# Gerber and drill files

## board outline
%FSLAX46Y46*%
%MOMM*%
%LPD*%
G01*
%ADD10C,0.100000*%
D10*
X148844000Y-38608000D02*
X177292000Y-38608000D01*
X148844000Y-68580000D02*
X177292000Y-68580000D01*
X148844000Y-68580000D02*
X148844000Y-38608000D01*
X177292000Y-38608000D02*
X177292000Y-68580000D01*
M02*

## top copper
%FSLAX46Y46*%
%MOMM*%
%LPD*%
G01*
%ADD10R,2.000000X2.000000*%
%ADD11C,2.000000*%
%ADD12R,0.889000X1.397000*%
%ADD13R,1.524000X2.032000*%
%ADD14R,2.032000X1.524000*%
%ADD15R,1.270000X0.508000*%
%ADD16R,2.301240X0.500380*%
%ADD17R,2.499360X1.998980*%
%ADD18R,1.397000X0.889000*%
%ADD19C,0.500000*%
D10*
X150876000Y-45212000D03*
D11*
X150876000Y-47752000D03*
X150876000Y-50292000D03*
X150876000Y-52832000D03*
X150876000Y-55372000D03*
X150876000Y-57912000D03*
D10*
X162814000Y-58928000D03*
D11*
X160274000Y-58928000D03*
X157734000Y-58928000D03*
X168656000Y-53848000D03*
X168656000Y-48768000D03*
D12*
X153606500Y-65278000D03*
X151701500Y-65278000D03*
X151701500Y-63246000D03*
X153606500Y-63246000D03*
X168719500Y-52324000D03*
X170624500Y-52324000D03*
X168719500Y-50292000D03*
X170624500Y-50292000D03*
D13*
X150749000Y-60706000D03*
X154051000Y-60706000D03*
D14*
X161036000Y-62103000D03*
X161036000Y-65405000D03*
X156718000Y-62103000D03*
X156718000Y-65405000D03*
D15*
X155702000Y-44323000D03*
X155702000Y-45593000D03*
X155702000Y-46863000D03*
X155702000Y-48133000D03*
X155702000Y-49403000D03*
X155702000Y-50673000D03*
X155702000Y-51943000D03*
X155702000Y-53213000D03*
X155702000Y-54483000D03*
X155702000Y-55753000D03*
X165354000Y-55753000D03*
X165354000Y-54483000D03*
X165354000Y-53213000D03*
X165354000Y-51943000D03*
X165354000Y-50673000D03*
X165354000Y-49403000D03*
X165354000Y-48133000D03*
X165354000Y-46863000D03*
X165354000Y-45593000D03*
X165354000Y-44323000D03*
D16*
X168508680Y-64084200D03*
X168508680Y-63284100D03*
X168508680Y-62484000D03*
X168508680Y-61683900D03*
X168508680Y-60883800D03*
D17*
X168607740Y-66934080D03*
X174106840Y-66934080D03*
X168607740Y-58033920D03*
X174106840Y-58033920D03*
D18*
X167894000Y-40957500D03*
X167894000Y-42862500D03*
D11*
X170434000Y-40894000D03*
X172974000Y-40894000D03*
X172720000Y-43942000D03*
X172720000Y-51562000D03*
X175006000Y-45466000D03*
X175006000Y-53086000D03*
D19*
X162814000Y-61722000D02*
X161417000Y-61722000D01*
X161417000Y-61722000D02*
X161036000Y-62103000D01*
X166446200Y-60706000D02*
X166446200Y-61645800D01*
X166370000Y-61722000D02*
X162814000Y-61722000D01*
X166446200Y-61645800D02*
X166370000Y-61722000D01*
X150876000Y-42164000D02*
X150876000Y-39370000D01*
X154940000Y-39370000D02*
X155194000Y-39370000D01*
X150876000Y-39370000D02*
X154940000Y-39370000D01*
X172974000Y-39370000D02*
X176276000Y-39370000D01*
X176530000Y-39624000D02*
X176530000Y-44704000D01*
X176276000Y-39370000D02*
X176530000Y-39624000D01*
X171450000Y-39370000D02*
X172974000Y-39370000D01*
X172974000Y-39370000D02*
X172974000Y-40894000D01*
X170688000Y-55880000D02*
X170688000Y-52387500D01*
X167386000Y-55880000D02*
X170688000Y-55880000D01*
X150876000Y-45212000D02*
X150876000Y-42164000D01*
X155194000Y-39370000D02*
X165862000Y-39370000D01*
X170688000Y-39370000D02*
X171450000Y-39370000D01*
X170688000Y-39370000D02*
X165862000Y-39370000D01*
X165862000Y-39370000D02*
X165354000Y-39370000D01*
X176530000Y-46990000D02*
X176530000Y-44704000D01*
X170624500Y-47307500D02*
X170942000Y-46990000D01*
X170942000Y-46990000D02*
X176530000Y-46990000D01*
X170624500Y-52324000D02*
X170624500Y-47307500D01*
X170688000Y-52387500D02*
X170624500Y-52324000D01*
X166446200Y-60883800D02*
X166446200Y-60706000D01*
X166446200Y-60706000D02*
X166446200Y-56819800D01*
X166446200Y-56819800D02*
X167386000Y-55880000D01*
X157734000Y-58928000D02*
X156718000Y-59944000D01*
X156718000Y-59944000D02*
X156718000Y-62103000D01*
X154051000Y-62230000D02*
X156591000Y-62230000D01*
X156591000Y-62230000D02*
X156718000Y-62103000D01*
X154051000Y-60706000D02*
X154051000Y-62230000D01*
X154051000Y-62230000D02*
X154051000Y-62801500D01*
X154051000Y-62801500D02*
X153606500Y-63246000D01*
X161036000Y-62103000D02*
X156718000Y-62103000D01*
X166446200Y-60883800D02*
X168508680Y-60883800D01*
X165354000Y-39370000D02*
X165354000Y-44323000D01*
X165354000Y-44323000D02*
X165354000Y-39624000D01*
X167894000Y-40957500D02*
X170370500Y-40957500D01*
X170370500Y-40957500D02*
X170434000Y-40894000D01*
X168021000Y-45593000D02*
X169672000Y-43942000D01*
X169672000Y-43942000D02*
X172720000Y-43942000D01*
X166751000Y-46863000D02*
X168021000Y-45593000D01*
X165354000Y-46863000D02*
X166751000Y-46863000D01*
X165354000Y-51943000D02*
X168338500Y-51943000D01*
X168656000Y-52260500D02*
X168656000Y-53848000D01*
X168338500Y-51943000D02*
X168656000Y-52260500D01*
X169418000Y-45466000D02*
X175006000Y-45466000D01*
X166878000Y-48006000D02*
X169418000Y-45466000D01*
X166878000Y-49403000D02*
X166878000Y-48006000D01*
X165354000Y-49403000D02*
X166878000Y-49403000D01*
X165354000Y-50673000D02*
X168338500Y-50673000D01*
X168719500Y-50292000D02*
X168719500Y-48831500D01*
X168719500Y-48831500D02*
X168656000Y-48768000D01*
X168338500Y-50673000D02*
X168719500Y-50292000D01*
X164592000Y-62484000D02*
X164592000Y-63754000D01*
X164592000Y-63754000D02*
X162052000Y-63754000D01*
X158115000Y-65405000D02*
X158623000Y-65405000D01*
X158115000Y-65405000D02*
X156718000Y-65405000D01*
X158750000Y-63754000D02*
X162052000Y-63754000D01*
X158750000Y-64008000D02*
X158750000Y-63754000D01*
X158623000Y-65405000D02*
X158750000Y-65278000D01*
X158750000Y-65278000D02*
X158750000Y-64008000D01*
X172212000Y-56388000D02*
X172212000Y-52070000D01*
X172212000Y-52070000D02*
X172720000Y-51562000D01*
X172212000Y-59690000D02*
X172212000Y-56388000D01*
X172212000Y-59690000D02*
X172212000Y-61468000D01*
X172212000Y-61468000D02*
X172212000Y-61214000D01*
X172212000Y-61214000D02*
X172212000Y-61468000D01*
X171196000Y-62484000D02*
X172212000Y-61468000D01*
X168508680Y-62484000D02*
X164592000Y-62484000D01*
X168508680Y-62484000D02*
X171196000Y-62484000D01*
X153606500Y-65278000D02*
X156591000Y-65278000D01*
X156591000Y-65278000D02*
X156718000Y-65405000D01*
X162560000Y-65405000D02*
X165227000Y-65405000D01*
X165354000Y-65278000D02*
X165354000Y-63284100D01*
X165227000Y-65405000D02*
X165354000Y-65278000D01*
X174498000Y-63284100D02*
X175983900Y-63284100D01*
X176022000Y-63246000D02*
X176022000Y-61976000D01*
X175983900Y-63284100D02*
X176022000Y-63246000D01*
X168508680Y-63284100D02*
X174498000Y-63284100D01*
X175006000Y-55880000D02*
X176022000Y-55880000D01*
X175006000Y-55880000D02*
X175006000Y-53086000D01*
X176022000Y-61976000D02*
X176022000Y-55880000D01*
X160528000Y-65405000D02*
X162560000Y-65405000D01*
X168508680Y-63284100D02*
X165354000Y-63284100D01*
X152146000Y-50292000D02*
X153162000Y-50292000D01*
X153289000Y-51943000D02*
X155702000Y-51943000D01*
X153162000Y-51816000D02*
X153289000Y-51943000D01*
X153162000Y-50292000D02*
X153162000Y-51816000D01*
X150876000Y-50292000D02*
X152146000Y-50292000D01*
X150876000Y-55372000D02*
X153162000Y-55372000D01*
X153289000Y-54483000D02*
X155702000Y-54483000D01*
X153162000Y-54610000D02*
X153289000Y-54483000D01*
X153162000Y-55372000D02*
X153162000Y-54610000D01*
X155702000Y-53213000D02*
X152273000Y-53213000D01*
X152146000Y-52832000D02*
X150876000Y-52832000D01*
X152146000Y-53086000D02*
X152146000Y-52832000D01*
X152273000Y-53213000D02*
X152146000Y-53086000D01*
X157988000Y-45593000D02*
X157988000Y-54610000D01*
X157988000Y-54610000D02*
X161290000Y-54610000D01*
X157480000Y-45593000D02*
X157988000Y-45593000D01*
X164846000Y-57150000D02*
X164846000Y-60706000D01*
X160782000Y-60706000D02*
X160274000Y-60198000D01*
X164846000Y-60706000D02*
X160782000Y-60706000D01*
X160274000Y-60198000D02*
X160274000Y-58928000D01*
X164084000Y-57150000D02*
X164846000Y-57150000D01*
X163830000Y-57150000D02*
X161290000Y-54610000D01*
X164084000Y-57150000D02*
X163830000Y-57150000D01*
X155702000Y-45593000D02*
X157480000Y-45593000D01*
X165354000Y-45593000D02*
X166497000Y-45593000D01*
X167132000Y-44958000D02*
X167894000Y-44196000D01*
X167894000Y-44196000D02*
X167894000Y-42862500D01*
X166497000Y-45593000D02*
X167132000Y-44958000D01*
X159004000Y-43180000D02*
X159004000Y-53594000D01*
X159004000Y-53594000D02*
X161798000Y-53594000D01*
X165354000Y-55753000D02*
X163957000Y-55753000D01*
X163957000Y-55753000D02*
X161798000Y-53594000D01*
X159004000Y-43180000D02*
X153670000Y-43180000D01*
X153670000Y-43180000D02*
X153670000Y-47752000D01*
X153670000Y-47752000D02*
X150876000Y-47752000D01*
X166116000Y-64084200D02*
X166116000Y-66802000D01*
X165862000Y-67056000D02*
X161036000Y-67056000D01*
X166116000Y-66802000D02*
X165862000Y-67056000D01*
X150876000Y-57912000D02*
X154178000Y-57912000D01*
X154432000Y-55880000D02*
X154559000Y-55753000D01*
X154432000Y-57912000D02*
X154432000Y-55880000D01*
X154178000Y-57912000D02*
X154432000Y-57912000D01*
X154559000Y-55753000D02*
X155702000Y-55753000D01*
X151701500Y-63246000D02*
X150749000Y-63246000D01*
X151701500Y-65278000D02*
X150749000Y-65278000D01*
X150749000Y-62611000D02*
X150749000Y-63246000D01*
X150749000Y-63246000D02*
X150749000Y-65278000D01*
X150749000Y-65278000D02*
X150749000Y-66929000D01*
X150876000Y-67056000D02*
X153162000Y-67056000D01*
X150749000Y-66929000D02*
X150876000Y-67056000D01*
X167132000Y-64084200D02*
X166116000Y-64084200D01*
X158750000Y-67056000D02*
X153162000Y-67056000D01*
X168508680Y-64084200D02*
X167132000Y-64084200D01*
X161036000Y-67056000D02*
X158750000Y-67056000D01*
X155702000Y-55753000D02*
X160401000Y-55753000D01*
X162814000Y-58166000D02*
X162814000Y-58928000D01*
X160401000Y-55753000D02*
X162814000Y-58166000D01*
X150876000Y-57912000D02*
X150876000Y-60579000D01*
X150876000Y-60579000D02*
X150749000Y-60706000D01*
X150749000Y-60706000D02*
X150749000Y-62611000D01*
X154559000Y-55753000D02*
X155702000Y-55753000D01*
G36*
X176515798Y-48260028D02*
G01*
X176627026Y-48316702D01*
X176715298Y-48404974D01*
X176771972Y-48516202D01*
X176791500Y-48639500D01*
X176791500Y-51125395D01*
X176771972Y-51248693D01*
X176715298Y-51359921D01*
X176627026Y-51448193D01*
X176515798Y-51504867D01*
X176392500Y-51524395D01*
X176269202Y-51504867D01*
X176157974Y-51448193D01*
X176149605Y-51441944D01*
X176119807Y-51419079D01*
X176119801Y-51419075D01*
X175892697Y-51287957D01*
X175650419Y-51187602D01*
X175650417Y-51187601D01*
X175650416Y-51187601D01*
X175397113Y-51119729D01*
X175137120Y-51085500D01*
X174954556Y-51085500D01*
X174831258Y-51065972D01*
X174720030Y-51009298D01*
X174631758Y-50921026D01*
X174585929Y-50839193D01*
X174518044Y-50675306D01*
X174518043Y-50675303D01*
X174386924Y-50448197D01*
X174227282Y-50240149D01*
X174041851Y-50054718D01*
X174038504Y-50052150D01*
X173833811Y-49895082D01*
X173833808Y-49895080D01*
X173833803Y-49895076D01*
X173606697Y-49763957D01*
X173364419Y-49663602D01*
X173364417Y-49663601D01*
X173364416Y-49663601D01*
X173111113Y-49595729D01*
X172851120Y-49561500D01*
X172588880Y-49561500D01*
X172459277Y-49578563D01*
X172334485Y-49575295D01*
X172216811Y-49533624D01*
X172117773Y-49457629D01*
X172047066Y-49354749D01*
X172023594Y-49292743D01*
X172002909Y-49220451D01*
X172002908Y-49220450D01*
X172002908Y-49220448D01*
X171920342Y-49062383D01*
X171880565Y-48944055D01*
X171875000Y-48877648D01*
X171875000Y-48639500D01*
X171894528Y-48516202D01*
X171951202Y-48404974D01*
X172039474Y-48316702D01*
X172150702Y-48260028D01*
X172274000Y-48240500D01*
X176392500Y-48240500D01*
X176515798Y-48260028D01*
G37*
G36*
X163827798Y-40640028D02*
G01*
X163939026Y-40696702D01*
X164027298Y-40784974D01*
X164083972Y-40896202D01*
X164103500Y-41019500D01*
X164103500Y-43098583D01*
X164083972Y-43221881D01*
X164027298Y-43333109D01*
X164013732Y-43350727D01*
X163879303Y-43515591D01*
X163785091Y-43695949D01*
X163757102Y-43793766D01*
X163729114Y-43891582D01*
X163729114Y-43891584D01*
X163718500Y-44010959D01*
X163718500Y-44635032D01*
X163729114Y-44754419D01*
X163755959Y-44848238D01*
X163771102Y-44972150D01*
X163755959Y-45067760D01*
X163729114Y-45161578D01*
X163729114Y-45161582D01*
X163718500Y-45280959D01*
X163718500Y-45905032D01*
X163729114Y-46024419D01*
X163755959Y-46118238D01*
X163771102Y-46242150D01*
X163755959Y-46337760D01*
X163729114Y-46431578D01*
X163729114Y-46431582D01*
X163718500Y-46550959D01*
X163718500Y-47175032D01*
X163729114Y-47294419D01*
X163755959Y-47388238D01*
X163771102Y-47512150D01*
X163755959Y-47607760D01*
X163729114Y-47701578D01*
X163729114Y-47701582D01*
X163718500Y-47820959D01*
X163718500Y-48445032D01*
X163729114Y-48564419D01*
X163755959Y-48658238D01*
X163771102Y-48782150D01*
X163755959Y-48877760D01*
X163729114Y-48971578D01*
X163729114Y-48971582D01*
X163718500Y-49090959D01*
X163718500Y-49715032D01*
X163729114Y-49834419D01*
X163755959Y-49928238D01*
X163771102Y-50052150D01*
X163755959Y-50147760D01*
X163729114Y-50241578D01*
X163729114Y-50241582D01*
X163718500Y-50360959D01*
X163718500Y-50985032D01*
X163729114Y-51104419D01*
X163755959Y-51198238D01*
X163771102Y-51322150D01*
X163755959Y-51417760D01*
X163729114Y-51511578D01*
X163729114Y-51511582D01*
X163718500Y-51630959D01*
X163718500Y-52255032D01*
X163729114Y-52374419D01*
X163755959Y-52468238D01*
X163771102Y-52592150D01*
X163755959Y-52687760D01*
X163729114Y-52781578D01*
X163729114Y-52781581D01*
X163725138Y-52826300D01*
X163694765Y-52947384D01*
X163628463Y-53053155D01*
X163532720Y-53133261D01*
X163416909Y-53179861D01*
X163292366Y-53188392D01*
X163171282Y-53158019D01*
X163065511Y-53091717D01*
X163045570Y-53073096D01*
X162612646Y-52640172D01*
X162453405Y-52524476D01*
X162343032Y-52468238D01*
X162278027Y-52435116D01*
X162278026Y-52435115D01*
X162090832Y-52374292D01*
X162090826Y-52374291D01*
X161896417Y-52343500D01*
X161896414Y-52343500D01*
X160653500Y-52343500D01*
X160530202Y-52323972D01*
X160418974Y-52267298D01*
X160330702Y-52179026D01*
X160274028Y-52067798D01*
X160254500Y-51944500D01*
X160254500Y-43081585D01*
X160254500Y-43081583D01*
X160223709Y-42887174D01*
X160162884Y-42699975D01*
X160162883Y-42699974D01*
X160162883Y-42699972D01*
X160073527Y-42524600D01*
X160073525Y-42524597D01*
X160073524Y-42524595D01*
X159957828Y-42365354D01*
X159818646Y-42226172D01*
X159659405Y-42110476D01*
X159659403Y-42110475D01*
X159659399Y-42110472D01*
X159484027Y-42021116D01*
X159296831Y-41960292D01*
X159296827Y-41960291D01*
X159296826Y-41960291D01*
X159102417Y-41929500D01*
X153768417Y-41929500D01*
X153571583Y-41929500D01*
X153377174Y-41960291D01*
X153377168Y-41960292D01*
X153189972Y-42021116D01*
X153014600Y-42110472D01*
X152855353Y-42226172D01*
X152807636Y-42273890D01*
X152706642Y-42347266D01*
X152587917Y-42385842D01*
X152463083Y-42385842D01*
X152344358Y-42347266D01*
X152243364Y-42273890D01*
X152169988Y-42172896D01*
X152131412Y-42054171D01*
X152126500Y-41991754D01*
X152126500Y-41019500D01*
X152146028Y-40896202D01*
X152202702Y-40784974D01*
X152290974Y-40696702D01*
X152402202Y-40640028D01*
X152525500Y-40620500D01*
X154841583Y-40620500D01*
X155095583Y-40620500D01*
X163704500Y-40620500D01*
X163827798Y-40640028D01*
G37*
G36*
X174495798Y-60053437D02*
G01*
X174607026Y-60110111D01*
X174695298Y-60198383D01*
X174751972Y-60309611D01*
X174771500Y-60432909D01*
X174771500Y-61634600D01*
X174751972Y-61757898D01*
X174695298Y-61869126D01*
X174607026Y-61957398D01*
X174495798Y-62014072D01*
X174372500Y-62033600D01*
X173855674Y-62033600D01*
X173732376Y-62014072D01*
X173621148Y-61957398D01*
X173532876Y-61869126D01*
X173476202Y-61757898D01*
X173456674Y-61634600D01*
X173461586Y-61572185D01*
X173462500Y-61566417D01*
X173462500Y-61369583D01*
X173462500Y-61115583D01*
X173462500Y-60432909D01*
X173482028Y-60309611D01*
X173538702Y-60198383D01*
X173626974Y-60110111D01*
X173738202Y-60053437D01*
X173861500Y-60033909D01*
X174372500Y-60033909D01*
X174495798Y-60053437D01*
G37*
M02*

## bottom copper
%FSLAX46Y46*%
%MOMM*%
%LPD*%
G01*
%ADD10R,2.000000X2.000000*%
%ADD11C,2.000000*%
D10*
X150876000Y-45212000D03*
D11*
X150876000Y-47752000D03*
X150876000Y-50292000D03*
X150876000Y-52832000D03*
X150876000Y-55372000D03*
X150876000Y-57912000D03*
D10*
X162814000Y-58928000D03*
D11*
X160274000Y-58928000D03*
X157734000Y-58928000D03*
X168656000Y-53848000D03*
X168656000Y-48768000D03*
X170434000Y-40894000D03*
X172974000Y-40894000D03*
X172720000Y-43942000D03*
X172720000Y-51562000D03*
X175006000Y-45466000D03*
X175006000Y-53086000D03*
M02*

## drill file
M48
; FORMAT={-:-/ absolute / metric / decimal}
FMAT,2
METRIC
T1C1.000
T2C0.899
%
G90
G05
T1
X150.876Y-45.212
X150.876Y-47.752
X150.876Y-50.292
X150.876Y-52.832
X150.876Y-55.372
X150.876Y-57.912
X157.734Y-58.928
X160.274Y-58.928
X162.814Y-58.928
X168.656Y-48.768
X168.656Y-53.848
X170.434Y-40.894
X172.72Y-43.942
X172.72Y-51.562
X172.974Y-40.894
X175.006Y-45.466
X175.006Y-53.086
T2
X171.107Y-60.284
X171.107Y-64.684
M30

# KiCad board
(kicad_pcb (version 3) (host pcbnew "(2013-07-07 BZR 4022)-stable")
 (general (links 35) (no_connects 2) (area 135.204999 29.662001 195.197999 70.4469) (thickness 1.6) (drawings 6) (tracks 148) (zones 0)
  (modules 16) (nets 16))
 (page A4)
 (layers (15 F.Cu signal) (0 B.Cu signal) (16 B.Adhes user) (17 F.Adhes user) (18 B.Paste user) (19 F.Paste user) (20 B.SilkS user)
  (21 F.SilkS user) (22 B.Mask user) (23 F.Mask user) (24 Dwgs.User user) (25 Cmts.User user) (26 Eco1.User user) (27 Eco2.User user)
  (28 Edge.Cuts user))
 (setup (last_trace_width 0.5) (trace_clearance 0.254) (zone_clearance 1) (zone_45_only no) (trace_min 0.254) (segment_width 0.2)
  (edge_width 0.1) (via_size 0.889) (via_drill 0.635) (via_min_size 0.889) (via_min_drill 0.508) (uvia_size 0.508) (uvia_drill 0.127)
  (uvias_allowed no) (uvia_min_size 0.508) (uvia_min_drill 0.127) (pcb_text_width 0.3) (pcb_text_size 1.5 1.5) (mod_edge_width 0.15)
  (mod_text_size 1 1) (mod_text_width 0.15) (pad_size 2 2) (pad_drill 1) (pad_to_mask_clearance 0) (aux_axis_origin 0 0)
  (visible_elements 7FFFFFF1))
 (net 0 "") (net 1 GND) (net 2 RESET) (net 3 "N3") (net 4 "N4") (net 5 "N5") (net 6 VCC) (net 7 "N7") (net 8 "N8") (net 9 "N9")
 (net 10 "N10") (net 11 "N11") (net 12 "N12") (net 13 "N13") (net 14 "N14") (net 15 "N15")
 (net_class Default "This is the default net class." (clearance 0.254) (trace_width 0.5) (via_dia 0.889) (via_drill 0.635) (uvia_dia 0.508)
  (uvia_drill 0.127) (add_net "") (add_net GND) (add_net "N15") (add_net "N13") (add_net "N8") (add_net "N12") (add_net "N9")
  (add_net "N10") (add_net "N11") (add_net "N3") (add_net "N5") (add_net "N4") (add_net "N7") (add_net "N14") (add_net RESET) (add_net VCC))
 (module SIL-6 (layer B.Cu) (at 150.876 51.562 270)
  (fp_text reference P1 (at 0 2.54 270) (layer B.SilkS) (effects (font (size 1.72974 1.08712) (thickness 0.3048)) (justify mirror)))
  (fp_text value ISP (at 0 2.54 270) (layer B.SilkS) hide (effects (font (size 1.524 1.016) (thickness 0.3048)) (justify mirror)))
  (pad 1 thru_hole rect (at -6.35 0 270) (size 2 2) (drill 1) (layers *.Cu *.Mask B.SilkS) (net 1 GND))
  (pad 2 thru_hole circle (at -3.81 0 270) (size 2 2) (drill 1) (layers *.Cu *.Mask B.SilkS) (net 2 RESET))
  (pad 3 thru_hole circle (at -1.27 0 270) (size 2 2) (drill 1) (layers *.Cu *.Mask B.SilkS) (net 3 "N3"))
  (pad 4 thru_hole circle (at 1.27 0 270) (size 2 2) (drill 1) (layers *.Cu *.Mask B.SilkS) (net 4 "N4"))
  (pad 5 thru_hole circle (at 3.81 0 270) (size 2 2) (drill 1) (layers *.Cu *.Mask B.SilkS) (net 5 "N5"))
  (pad 6 thru_hole circle (at 6.35 0 270) (size 2 2) (drill 1) (layers *.Cu *.Mask B.SilkS) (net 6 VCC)))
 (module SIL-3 (layer B.Cu) (at 160.274 58.928 180)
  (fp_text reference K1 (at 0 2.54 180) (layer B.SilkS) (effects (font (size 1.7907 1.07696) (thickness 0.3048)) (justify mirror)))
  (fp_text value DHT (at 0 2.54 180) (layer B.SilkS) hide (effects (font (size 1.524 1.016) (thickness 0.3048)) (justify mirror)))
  (pad 1 thru_hole rect (at -2.54 0 180) (size 2 2) (drill 1) (layers *.Cu *.Mask B.SilkS) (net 6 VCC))
  (pad 2 thru_hole circle (at 0 0 180) (size 2 2) (drill 1) (layers *.Cu *.Mask B.SilkS) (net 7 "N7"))
  (pad 3 thru_hole circle (at 2.54 0 180) (size 2 2) (drill 1) (layers *.Cu *.Mask B.SilkS) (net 1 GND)))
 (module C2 (layer B.Cu) (at 168.656 51.308 90)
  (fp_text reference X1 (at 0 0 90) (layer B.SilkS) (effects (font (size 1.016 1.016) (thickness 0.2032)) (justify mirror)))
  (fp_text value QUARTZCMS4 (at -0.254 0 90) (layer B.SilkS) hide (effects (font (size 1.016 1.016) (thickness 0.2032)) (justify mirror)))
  (pad 1 thru_hole circle (at -2.54 0 90) (size 2 2) (drill 1) (layers *.Cu *.Mask B.SilkS) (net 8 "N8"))
  (pad 3 thru_hole circle (at 2.54 0 90) (size 2 2) (drill 1) (layers *.Cu *.Mask B.SilkS) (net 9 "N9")))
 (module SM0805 (layer F.Cu) (at 152.654 65.278 180)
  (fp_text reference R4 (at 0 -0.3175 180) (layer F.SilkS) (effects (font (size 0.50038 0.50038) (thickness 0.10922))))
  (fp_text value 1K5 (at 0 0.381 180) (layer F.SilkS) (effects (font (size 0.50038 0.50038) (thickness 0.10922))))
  (pad 1 smd rect (at -0.9525 0 180) (size 0.889 1.397) (layers F.Cu F.Paste F.Mask) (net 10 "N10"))
  (pad 2 smd rect (at 0.9525 0 180) (size 0.889 1.397) (layers F.Cu F.Paste F.Mask) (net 6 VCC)))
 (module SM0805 (layer F.Cu) (at 152.654 63.246)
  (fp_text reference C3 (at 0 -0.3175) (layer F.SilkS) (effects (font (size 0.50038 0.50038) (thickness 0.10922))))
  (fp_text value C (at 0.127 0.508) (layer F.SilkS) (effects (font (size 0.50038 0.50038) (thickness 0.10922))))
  (pad 1 smd rect (at -0.9525 0) (size 0.889 1.397) (layers F.Cu F.Paste F.Mask) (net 6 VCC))
  (pad 2 smd rect (at 0.9525 0) (size 0.889 1.397) (layers F.Cu F.Paste F.Mask) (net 1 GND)))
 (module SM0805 (layer F.Cu) (at 169.672 52.324)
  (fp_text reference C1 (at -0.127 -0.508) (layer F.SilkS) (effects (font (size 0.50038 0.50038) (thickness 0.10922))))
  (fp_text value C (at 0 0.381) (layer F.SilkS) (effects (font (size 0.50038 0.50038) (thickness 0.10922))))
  (pad 1 smd rect (at -0.9525 0) (size 0.889 1.397) (layers F.Cu F.Paste F.Mask) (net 8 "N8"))
  (pad 2 smd rect (at 0.9525 0) (size 0.889 1.397) (layers F.Cu F.Paste F.Mask) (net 1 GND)))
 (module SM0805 (layer F.Cu) (at 169.672 50.292)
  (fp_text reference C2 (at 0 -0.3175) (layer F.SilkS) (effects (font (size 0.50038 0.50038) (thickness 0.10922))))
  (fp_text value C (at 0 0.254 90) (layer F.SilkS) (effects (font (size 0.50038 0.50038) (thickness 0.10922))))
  (pad 1 smd rect (at -0.9525 0) (size 0.889 1.397) (layers F.Cu F.Paste F.Mask) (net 9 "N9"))
  (pad 2 smd rect (at 0.9525 0) (size 0.889 1.397) (layers F.Cu F.Paste F.Mask) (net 1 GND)))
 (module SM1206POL (layer F.Cu) (at 152.4 60.706)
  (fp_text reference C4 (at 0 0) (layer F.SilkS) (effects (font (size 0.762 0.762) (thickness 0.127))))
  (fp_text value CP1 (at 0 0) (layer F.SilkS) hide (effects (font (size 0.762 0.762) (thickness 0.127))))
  (pad 1 smd rect (at -1.651 0) (size 1.524 2.032) (layers F.Cu F.Paste F.Mask) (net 6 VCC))
  (pad 2 smd rect (at 1.651 0) (size 1.524 2.032) (layers F.Cu F.Paste F.Mask) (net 1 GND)))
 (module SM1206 (layer F.Cu) (at 161.036 63.754 270)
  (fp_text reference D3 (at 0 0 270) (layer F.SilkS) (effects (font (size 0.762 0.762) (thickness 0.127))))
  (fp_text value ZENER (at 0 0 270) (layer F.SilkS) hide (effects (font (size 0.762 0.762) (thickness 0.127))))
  (pad 1 smd rect (at -1.651 0 270) (size 1.524 2.032) (layers F.Cu F.Paste F.Mask) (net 1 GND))
  (pad 2 smd rect (at 1.651 0 270) (size 1.524 2.032) (layers F.Cu F.Paste F.Mask) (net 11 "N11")))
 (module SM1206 (layer F.Cu) (at 156.718 63.754 270)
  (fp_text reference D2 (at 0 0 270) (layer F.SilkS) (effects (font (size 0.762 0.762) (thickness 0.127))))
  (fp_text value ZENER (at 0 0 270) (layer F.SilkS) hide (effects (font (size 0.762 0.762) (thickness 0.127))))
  (pad 1 smd rect (at -1.651 0 270) (size 1.524 2.032) (layers F.Cu F.Paste F.Mask) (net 1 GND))
  (pad 2 smd rect (at 1.651 0 270) (size 1.524 2.032) (layers F.Cu F.Paste F.Mask) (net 10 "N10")))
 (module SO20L (layer F.Cu) (at 160.528 50.038 90)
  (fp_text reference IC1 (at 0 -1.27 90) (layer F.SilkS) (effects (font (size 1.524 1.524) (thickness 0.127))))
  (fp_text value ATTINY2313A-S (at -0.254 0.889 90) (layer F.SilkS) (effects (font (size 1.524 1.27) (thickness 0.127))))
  (pad 11 smd rect (at 5.715 -4.826 90) (size 0.508 1.27) (layers F.Cu F.Paste F.Mask))
  (pad 12 smd rect (at 4.445 -4.826 90) (size 0.508 1.27) (layers F.Cu F.Paste F.Mask) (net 7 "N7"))
  (pad 13 smd rect (at 3.175 -4.826 90) (size 0.508 1.27) (layers F.Cu F.Paste F.Mask))
  (pad 14 smd rect (at 1.905 -4.826 90) (size 0.508 1.27) (layers F.Cu F.Paste F.Mask))
  (pad 15 smd rect (at 0.635 -4.826 90) (size 0.508 1.27) (layers F.Cu F.Paste F.Mask))
  (pad 16 smd rect (at -0.635 -4.826 90) (size 0.508 1.27) (layers F.Cu F.Paste F.Mask))
  (pad 17 smd rect (at -1.905 -4.826 90) (size 0.508 1.27) (layers F.Cu F.Paste F.Mask) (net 3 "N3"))
  (pad 18 smd rect (at -3.175 -4.826 90) (size 0.508 1.27) (layers F.Cu F.Paste F.Mask) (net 4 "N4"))
  (pad 19 smd rect (at -4.445 -4.826 90) (size 0.508 1.27) (layers F.Cu F.Paste F.Mask) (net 5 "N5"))
  (pad 20 smd rect (at -5.715 -4.826 90) (size 0.508 1.27) (layers F.Cu F.Paste F.Mask) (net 6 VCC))
  (pad 1 smd rect (at -5.715 4.826 90) (size 0.508 1.27) (layers F.Cu F.Paste F.Mask) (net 2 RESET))
  (pad 2 smd rect (at -4.445 4.826 90) (size 0.508 1.27) (layers F.Cu F.Paste F.Mask))
  (pad 3 smd rect (at -3.175 4.826 90) (size 0.508 1.27) (layers F.Cu F.Paste F.Mask))
  (pad 4 smd rect (at -1.905 4.826 90) (size 0.508 1.27) (layers F.Cu F.Paste F.Mask) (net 8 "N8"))
  (pad 5 smd rect (at -0.635 4.826 90) (size 0.508 1.27) (layers F.Cu F.Paste F.Mask) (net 9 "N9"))
  (pad 6 smd rect (at 0.635 4.826 90) (size 0.508 1.27) (layers F.Cu F.Paste F.Mask) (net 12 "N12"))
  (pad 7 smd rect (at 1.905 4.826 90) (size 0.508 1.27) (layers F.Cu F.Paste F.Mask))
  (pad 8 smd rect (at 3.175 4.826 90) (size 0.508 1.27) (layers F.Cu F.Paste F.Mask) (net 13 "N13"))
  (pad 9 smd rect (at 4.445 4.826 90) (size 0.508 1.27) (layers F.Cu F.Paste F.Mask) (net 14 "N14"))
  (pad 10 smd rect (at 5.715 4.826 90) (size 0.508 1.27) (layers F.Cu F.Paste F.Mask) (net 1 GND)))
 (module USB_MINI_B (layer F.Cu) (at 171.958 62.484 180)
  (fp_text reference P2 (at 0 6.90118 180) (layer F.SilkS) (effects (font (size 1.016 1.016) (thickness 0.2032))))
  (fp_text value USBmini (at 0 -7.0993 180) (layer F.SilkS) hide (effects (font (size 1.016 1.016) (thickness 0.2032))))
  (pad 1 smd rect (at 3.44932 -1.6002 180) (size 2.30124 0.50038) (layers F.Cu F.Paste F.Mask) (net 6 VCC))
  (pad 2 smd rect (at 3.44932 -0.8001 180) (size 2.30124 0.50038) (layers F.Cu F.Paste F.Mask) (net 11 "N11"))
  (pad 3 smd rect (at 3.44932 0 180) (size 2.30124 0.50038) (layers F.Cu F.Paste F.Mask) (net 10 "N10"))
  (pad 4 smd rect (at 3.44932 0.8001 180) (size 2.30124 0.50038) (layers F.Cu F.Paste F.Mask))
  (pad 5 smd rect (at 3.44932 1.6002 180) (size 2.30124 0.50038) (layers F.Cu F.Paste F.Mask) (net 1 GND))
  (pad 6 smd rect (at 3.35026 -4.45008 180) (size 2.49936 1.99898) (layers F.Cu F.Paste F.Mask))
  (pad 7 smd rect (at -2.14884 -4.45008 180) (size 2.49936 1.99898) (layers F.Cu F.Paste F.Mask))
  (pad 8 smd rect (at 3.35026 4.45008 180) (size 2.49936 1.99898) (layers F.Cu F.Paste F.Mask))
  (pad 9 smd rect (at -2.14884 4.45008 180) (size 2.49936 1.99898) (layers F.Cu F.Paste F.Mask))
  (pad "" np_thru_hole circle (at 0.8509 -2.19964 180) (size 0.89916 0.89916) (drill 0.89916) (layers *.Cu *.Mask F.SilkS))
  (pad 2 np_thru_hole circle (at 0.8509 2.19964 180) (size 0.89916 0.89916) (drill 0.89916) (layers *.Cu *.Mask F.SilkS) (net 11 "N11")))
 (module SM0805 (layer F.Cu) (at 167.894 41.91 270)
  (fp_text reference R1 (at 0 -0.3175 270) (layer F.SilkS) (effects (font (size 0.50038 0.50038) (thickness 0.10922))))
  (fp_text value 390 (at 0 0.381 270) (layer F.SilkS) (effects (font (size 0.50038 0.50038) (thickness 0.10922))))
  (pad 1 smd rect (at -0.9525 0 270) (size 0.889 1.397) (layers F.Cu F.Paste F.Mask) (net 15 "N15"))
  (pad 2 smd rect (at 0.9525 0 270) (size 0.889 1.397) (layers F.Cu F.Paste F.Mask) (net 14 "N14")))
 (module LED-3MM (layer B.Cu) (at 171.704 40.894)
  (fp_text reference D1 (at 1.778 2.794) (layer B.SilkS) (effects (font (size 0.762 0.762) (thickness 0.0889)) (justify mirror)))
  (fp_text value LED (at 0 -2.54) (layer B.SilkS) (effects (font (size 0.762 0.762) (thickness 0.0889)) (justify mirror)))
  (pad 1 thru_hole circle (at -1.27 0) (size 2 2) (drill 1) (layers *.Cu *.Mask B.SilkS) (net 15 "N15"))
  (pad 2 thru_hole circle (at 1.27 0) (size 2 2) (drill 1) (layers *.Cu *.Mask B.SilkS) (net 1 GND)))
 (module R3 (layer B.Cu) (at 172.72 47.752 270) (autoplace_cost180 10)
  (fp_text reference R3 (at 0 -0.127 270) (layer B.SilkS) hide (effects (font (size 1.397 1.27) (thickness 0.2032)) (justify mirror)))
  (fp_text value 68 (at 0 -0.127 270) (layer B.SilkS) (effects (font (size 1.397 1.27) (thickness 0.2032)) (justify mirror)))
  (pad 1 thru_hole circle (at -3.81 0 270) (size 2 2) (drill 1) (layers *.Cu *.Mask B.SilkS) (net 13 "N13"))
  (pad 2 thru_hole circle (at 3.81 0 270) (size 2 2) (drill 1) (layers *.Cu *.Mask B.SilkS) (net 10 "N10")))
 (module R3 (layer B.Cu) (at 175.006 49.276 270) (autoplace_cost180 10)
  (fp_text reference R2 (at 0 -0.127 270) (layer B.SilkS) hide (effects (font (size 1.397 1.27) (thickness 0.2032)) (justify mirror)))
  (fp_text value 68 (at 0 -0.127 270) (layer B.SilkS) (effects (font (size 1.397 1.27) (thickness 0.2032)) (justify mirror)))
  (pad 1 thru_hole circle (at -3.81 0 270) (size 2 2) (drill 1) (layers *.Cu *.Mask B.SilkS) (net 12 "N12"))
  (pad 2 thru_hole circle (at 3.81 0 270) (size 2 2) (drill 1) (layers *.Cu *.Mask B.SilkS) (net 11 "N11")))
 (gr_line (start 148.844 38.608) (end 177.292 38.608) (angle 90) (layer Edge.Cuts) (width 0.1))
 (gr_line (start 148.844 68.58) (end 177.292 68.58) (angle 90) (layer Edge.Cuts) (width 0.1))
 (gr_line (start 148.844 68.58) (end 148.844 38.608) (angle 90) (layer Edge.Cuts) (width 0.1))
 (gr_line (start 177.292 38.608) (end 177.292 68.58) (angle 90) (layer Edge.Cuts) (width 0.1))
 (segment (start 162.814 61.722) (end 161.417 61.722) (width 0.5) (layer F.Cu) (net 1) (status 800000))
 (segment (start 161.417 61.722) (end 161.036 62.103) (width 0.5) (layer F.Cu) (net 1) (status C00000))
 (segment (start 166.4462 60.706) (end 166.4462 61.6458) (width 0.5) (layer F.Cu) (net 1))
 (segment (start 166.37 61.722) (end 162.814 61.722) (width 0.5) (layer F.Cu) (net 1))
 (segment (start 166.4462 61.6458) (end 166.37 61.722) (width 0.5) (layer F.Cu) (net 1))
 (segment (start 150.876 42.164) (end 150.876 39.37) (width 0.5) (layer F.Cu) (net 1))
 (segment (start 154.94 39.37) (end 155.194 39.37) (width 0.5) (layer F.Cu) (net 1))
 (segment (start 150.876 39.37) (end 154.94 39.37) (width 0.5) (layer F.Cu) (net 1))
 (segment (start 172.974 39.37) (end 176.276 39.37) (width 0.5) (layer F.Cu) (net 1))
 (segment (start 176.53 39.624) (end 176.53 44.704) (width 0.5) (layer F.Cu) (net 1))
 (segment (start 176.276 39.37) (end 176.53 39.624) (width 0.5) (layer F.Cu) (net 1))
 (segment (start 171.45 39.37) (end 172.974 39.37) (width 0.5) (layer F.Cu) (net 1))
 (segment (start 172.974 39.37) (end 172.974 40.894) (width 0.5) (layer F.Cu) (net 1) (status 800000))
 (segment (start 170.688 55.88) (end 170.688 52.3875) (width 0.5) (layer F.Cu) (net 1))
 (segment (start 167.386 55.88) (end 170.688 55.88) (width 0.5) (layer F.Cu) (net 1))
 (segment (start 150.876 45.212) (end 150.876 42.164) (width 0.5) (layer F.Cu) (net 1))
 (segment (start 155.194 39.37) (end 165.862 39.37) (width 0.5) (layer F.Cu) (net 1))
 (segment (start 170.688 39.37) (end 171.45 39.37) (width 0.5) (layer F.Cu) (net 1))
 (segment (start 170.688 39.37) (end 165.862 39.37) (width 0.5) (layer F.Cu) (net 1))
 (segment (start 165.862 39.37) (end 165.354 39.37) (width 0.5) (layer F.Cu) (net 1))
 (segment (start 176.53 46.99) (end 176.53 44.704) (width 0.5) (layer F.Cu) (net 1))
 (segment (start 170.6245 47.3075) (end 170.942 46.99) (width 0.5) (layer F.Cu) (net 1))
 (segment (start 170.942 46.99) (end 176.53 46.99) (width 0.5) (layer F.Cu) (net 1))
 (segment (start 170.6245 52.324) (end 170.6245 47.3075) (width 0.5) (layer F.Cu) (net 1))
 (segment (start 170.688 52.3875) (end 170.6245 52.324) (width 0.5) (layer F.Cu) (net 1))
 (segment (start 166.4462 60.8838) (end 166.4462 60.706) (width 0.5) (layer F.Cu) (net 1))
 (segment (start 166.4462 60.706) (end 166.4462 56.8198) (width 0.5) (layer F.Cu) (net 1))
 (segment (start 166.4462 56.8198) (end 167.386 55.88) (width 0.5) (layer F.Cu) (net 1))
 (segment (start 157.734 58.928) (end 156.718 59.944) (width 0.5) (layer F.Cu) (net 1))
 (segment (start 156.718 59.944) (end 156.718 62.103) (width 0.5) (layer F.Cu) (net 1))
 (segment (start 154.051 62.23) (end 156.591 62.23) (width 0.5) (layer F.Cu) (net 1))
 (segment (start 156.591 62.23) (end 156.718 62.103) (width 0.5) (layer F.Cu) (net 1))
 (segment (start 154.051 60.706) (end 154.051 62.23) (width 0.5) (layer F.Cu) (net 1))
 (segment (start 154.051 62.23) (end 154.051 62.8015) (width 0.5) (layer F.Cu) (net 1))
 (segment (start 154.051 62.8015) (end 153.6065 63.246) (width 0.5) (layer F.Cu) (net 1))
 (segment (start 161.036 62.103) (end 156.718 62.103) (width 0.5) (layer F.Cu) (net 1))
 (segment (start 166.4462 60.8838) (end 168.50868 60.8838) (width 0.5) (layer F.Cu) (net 1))
 (segment (start 165.354 39.37) (end 165.354 44.323) (width 0.5) (layer F.Cu) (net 1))
 (segment (start 165.354 44.323) (end 165.354 39.624) (width 0.5) (layer F.Cu) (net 1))
 (segment (start 167.894 40.9575) (end 170.3705 40.9575) (width 0.5) (layer F.Cu) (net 15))
 (segment (start 170.3705 40.9575) (end 170.434 40.894) (width 0.5) (layer F.Cu) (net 15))
 (segment (start 168.021 45.593) (end 169.672 43.942) (width 0.5) (layer F.Cu) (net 13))
 (segment (start 169.672 43.942) (end 172.72 43.942) (width 0.5) (layer F.Cu) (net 13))
 (segment (start 166.751 46.863) (end 168.021 45.593) (width 0.5) (layer F.Cu) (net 13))
 (segment (start 165.354 46.863) (end 166.751 46.863) (width 0.5) (layer F.Cu) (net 13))
 (segment (start 165.354 51.943) (end 168.3385 51.943) (width 0.5) (layer F.Cu) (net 8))
 (segment (start 168.656 52.2605) (end 168.656 53.848) (width 0.5) (layer F.Cu) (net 8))
 (segment (start 168.3385 51.943) (end 168.656 52.2605) (width 0.5) (layer F.Cu) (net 8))
 (segment (start 169.418 45.466) (end 175.006 45.466) (width 0.5) (layer F.Cu) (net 12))
 (segment (start 166.878 48.006) (end 169.418 45.466) (width 0.5) (layer F.Cu) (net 12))
 (segment (start 166.878 49.403) (end 166.878 48.006) (width 0.5) (layer F.Cu) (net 12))
 (segment (start 165.354 49.403) (end 166.878 49.403) (width 0.5) (layer F.Cu) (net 12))
 (segment (start 165.354 50.673) (end 168.3385 50.673) (width 0.5) (layer F.Cu) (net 9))
 (segment (start 168.7195 50.292) (end 168.7195 48.8315) (width 0.5) (layer F.Cu) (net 9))
 (segment (start 168.7195 48.8315) (end 168.656 48.768) (width 0.5) (layer F.Cu) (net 9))
 (segment (start 168.3385 50.673) (end 168.7195 50.292) (width 0.5) (layer F.Cu) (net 9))
 (segment (start 164.592 62.484) (end 164.592 63.754) (width 0.5) (layer F.Cu) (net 10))
 (segment (start 164.592 63.754) (end 162.052 63.754) (width 0.5) (layer F.Cu) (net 10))
 (segment (start 158.115 65.405) (end 158.623 65.405) (width 0.5) (layer F.Cu) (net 10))
 (segment (start 158.115 65.405) (end 156.718 65.405) (width 0.5) (layer F.Cu) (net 10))
 (segment (start 158.75 63.754) (end 162.052 63.754) (width 0.5) (layer F.Cu) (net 10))
 (segment (start 158.75 64.008) (end 158.75 63.754) (width 0.5) (layer F.Cu) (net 10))
 (segment (start 158.623 65.405) (end 158.75 65.278) (width 0.5) (layer F.Cu) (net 10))
 (segment (start 158.75 65.278) (end 158.75 64.008) (width 0.5) (layer F.Cu) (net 10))
 (segment (start 172.212 56.388) (end 172.212 52.07) (width 0.5) (layer F.Cu) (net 10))
 (segment (start 172.212 52.07) (end 172.72 51.562) (width 0.5) (layer F.Cu) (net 10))
 (segment (start 172.212 59.69) (end 172.212 56.388) (width 0.5) (layer F.Cu) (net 10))
 (segment (start 172.212 59.69) (end 172.212 61.468) (width 0.5) (layer F.Cu) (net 10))
 (segment (start 172.212 61.468) (end 172.212 61.214) (width 0.5) (layer F.Cu) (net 10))
 (segment (start 172.212 61.214) (end 172.212 61.468) (width 0.5) (layer F.Cu) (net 10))
 (segment (start 171.196 62.484) (end 172.212 61.468) (width 0.5) (layer F.Cu) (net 10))
 (segment (start 168.50868 62.484) (end 164.592 62.484) (width 0.5) (layer F.Cu) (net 10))
 (segment (start 168.50868 62.484) (end 171.196 62.484) (width 0.5) (layer F.Cu) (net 10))
 (segment (start 153.6065 65.278) (end 156.591 65.278) (width 0.5) (layer F.Cu) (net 10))
 (segment (start 156.591 65.278) (end 156.718 65.405) (width 0.5) (layer F.Cu) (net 10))
 (segment (start 162.56 65.405) (end 165.227 65.405) (width 0.5) (layer F.Cu) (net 11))
 (segment (start 165.354 65.278) (end 165.354 63.2841) (width 0.5) (layer F.Cu) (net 11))
 (segment (start 165.227 65.405) (end 165.354 65.278) (width 0.5) (layer F.Cu) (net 11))
 (segment (start 174.498 63.2841) (end 175.9839 63.2841) (width 0.5) (layer F.Cu) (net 11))
 (segment (start 176.022 63.246) (end 176.022 61.976) (width 0.5) (layer F.Cu) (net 11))
 (segment (start 175.9839 63.2841) (end 176.022 63.246) (width 0.5) (layer F.Cu) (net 11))
 (segment (start 168.50868 63.2841) (end 174.498 63.2841) (width 0.5) (layer F.Cu) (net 11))
 (segment (start 175.006 55.88) (end 176.022 55.88) (width 0.5) (layer F.Cu) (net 11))
 (segment (start 175.006 55.88) (end 175.006 53.086) (width 0.5) (layer F.Cu) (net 11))
 (segment (start 176.022 61.976) (end 176.022 55.88) (width 0.5) (layer F.Cu) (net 11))
 (segment (start 160.528 65.405) (end 162.56 65.405) (width 0.5) (layer F.Cu) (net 11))
 (segment (start 168.50868 63.2841) (end 165.354 63.2841) (width 0.5) (layer F.Cu) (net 11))
 (segment (start 152.146 50.292) (end 153.162 50.292) (width 0.5) (layer F.Cu) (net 3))
 (segment (start 153.289 51.943) (end 155.702 51.943) (width 0.5) (layer F.Cu) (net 3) (status 800000))
 (segment (start 153.162 51.816) (end 153.289 51.943) (width 0.5) (layer F.Cu) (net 3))
 (segment (start 153.162 50.292) (end 153.162 51.816) (width 0.5) (layer F.Cu) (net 3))
 (segment (start 150.876 50.292) (end 152.146 50.292) (width 0.5) (layer F.Cu) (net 3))
 (segment (start 150.876 55.372) (end 153.162 55.372) (width 0.5) (layer F.Cu) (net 5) (status 400000))
 (segment (start 153.289 54.483) (end 155.702 54.483) (width 0.5) (layer F.Cu) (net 5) (status 800000))
 (segment (start 153.162 54.61) (end 153.289 54.483) (width 0.5) (layer F.Cu) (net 5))
 (segment (start 153.162 55.372) (end 153.162 54.61) (width 0.5) (layer F.Cu) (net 5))
 (segment (start 155.702 53.213) (end 152.273 53.213) (width 0.5) (layer F.Cu) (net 4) (status 400000))
 (segment (start 152.146 52.832) (end 150.876 52.832) (width 0.5) (layer F.Cu) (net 4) (status 800000))
 (segment (start 152.146 53.086) (end 152.146 52.832) (width 0.5) (layer F.Cu) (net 4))
 (segment (start 152.273 53.213) (end 152.146 53.086) (width 0.5) (layer F.Cu) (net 4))
 (segment (start 157.988 45.593) (end 157.988 54.61) (width 0.5) (layer F.Cu) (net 7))
 (segment (start 157.988 54.61) (end 161.29 54.61) (width 0.5) (layer F.Cu) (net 7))
 (segment (start 157.48 45.593) (end 157.988 45.593) (width 0.5) (layer F.Cu) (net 7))
 (segment (start 164.846 57.15) (end 164.846 60.706) (width 0.5) (layer F.Cu) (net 7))
 (segment (start 160.782 60.706) (end 160.274 60.198) (width 0.5) (layer F.Cu) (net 7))
 (segment (start 164.846 60.706) (end 160.782 60.706) (width 0.5) (layer F.Cu) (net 7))
 (segment (start 160.274 60.198) (end 160.274 58.928) (width 0.5) (layer F.Cu) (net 7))
 (segment (start 164.084 57.15) (end 164.846 57.15) (width 0.5) (layer F.Cu) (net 7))
 (segment (start 163.83 57.15) (end 161.29 54.61) (width 0.5) (layer F.Cu) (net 7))
 (segment (start 164.084 57.15) (end 163.83 57.15) (width 0.5) (layer F.Cu) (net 7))
 (segment (start 155.702 45.593) (end 157.48 45.593) (width 0.5) (layer F.Cu) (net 7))
 (segment (start 165.354 45.593) (end 166.497 45.593) (width 0.5) (layer F.Cu) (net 14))
 (segment (start 167.132 44.958) (end 167.894 44.196) (width 0.5) (layer F.Cu) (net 14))
 (segment (start 167.894 44.196) (end 167.894 42.8625) (width 0.5) (layer F.Cu) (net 14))
 (segment (start 166.497 45.593) (end 167.132 44.958) (width 0.5) (layer F.Cu) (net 14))
 (segment (start 159.004 43.18) (end 159.004 53.594) (width 0.5) (layer F.Cu) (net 2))
 (segment (start 159.004 53.594) (end 161.798 53.594) (width 0.5) (layer F.Cu) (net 2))
 (segment (start 165.354 55.753) (end 163.957 55.753) (width 0.5) (layer F.Cu) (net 2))
 (segment (start 163.957 55.753) (end 161.798 53.594) (width 0.5) (layer F.Cu) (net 2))
 (segment (start 159.004 43.18) (end 153.67 43.18) (width 0.5) (layer F.Cu) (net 2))
 (segment (start 153.67 43.18) (end 153.67 47.752) (width 0.5) (layer F.Cu) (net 2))
 (segment (start 153.67 47.752) (end 150.876 47.752) (width 0.5) (layer F.Cu) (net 2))
 (segment (start 166.116 64.0842) (end 166.116 66.802) (width 0.5) (layer F.Cu) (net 6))
 (segment (start 165.862 67.056) (end 161.036 67.056) (width 0.5) (layer F.Cu) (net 6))
 (segment (start 166.116 66.802) (end 165.862 67.056) (width 0.5) (layer F.Cu) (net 6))
 (segment (start 150.876 57.912) (end 154.178 57.912) (width 0.5) (layer F.Cu) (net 6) (status 400000))
 (segment (start 154.432 55.88) (end 154.559 55.753) (width 0.5) (layer F.Cu) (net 6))
 (segment (start 154.432 57.912) (end 154.432 55.88) (width 0.5) (layer F.Cu) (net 6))
 (segment (start 154.178 57.912) (end 154.432 57.912) (width 0.5) (layer F.Cu) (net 6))
 (segment (start 154.559 55.753) (end 155.702 55.753) (width 0.5) (layer F.Cu) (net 6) (status 800000))
 (segment (start 151.7015 63.246) (end 150.749 63.246) (width 0.5) (layer F.Cu) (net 6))
 (segment (start 151.7015 65.278) (end 150.749 65.278) (width 0.5) (layer F.Cu) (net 6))
 (segment (start 150.749 62.611) (end 150.749 63.246) (width 0.5) (layer F.Cu) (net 6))
 (segment (start 150.749 63.246) (end 150.749 65.278) (width 0.5) (layer F.Cu) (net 6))
 (segment (start 150.749 65.278) (end 150.749 66.929) (width 0.5) (layer F.Cu) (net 6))
 (segment (start 150.876 67.056) (end 153.162 67.056) (width 0.5) (layer F.Cu) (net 6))
 (segment (start 150.749 66.929) (end 150.876 67.056) (width 0.5) (layer F.Cu) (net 6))
 (segment (start 167.132 64.0842) (end 166.116 64.0842) (width 0.5) (layer F.Cu) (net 6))
 (segment (start 158.75 67.056) (end 153.162 67.056) (width 0.5) (layer F.Cu) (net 6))
 (segment (start 168.50868 64.0842) (end 167.132 64.0842) (width 0.5) (layer F.Cu) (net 6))
 (segment (start 161.036 67.056) (end 158.75 67.056) (width 0.5) (layer F.Cu) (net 6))
 (segment (start 155.702 55.753) (end 160.401 55.753) (width 0.5) (layer F.Cu) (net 6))
 (segment (start 162.814 58.166) (end 162.814 58.928) (width 0.5) (layer F.Cu) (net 6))
 (segment (start 160.401 55.753) (end 162.814 58.166) (width 0.5) (layer F.Cu) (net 6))
 (segment (start 150.876 57.912) (end 150.876 60.579) (width 0.5) (layer F.Cu) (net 6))
 (segment (start 150.876 60.579) (end 150.749 60.706) (width 0.5) (layer F.Cu) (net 6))
 (segment (start 150.749 60.706) (end 150.749 62.611) (width 0.5) (layer F.Cu) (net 6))
 (segment (start 154.559 55.753) (end 155.702 55.753) (width 0.5) (layer F.Cu) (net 6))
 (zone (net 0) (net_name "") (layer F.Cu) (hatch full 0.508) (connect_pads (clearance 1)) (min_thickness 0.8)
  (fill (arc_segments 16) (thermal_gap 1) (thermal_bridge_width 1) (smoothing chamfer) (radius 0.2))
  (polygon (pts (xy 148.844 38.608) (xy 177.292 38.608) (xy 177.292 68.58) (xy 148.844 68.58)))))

